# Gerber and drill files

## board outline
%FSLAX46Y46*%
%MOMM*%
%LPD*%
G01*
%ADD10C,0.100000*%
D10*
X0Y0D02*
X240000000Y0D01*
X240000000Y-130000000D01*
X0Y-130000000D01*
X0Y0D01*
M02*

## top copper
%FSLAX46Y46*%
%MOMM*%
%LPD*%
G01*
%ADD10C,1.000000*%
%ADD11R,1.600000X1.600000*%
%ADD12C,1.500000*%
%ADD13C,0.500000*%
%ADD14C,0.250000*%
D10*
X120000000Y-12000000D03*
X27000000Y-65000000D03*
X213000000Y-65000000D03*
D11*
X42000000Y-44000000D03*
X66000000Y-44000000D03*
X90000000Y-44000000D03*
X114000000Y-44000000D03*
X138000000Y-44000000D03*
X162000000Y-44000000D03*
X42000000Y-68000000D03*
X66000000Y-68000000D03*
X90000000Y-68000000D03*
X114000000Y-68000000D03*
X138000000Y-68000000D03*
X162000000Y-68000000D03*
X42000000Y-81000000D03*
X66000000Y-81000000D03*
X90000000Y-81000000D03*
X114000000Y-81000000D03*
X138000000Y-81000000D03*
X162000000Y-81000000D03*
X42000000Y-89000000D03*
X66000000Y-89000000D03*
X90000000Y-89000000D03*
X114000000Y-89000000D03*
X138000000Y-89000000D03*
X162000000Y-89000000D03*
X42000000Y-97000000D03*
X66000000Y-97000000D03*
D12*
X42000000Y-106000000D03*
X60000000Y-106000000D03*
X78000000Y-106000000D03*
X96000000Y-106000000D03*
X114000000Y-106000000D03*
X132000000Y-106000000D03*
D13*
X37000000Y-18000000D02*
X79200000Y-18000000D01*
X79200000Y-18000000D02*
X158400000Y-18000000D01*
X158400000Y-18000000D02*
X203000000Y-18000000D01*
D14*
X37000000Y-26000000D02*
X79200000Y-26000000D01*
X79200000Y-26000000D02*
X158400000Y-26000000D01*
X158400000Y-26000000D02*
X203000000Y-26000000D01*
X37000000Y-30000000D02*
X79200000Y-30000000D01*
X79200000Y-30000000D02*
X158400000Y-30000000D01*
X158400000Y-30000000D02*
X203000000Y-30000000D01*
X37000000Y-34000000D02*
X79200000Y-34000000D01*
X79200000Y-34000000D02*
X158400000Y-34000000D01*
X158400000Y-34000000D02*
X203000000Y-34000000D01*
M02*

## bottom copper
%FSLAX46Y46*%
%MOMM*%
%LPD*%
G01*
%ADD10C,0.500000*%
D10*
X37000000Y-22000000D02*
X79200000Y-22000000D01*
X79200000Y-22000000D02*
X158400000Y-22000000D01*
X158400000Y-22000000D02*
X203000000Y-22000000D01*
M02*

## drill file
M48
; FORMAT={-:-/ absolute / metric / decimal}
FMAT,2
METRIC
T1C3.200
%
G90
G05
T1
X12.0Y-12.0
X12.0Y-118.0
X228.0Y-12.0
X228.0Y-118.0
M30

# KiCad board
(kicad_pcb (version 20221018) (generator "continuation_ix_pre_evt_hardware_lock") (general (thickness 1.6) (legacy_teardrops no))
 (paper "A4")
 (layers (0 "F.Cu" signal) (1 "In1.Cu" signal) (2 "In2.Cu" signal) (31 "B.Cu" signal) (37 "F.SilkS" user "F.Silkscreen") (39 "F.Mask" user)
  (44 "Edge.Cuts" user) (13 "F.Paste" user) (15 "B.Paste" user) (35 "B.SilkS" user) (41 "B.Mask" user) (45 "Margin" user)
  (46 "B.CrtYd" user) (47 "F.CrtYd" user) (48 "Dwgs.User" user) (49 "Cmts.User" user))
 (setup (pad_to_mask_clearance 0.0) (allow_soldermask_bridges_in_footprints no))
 (gr_rect (start 0 0) (end 240.0 130.0) (stroke (width 0.1) (type default)) (fill none) (layer "Edge.Cuts"))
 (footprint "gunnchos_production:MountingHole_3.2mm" (layer "F.Cu") (at 12.0 12.0)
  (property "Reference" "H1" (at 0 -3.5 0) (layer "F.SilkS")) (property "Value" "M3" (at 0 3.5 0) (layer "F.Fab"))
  (pad "" np_thru_hole circle (at 0 0) (size 3.2 3.2) (drill 3.2) (layers "*.Cu" "*.Mask")))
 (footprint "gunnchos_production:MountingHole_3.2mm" (layer "F.Cu") (at 228.0 12.0)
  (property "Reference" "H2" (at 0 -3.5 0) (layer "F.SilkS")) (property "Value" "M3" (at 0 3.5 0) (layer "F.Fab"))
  (pad "" np_thru_hole circle (at 0 0) (size 3.2 3.2) (drill 3.2) (layers "*.Cu" "*.Mask")))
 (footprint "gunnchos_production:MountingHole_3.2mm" (layer "F.Cu") (at 12.0 118.0)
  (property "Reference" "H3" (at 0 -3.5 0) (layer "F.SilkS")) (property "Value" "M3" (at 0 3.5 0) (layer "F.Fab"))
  (pad "" np_thru_hole circle (at 0 0) (size 3.2 3.2) (drill 3.2) (layers "*.Cu" "*.Mask")))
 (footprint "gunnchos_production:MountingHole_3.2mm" (layer "F.Cu") (at 228.0 118.0)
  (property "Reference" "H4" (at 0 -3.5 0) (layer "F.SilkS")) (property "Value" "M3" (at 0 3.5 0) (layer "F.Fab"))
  (pad "" np_thru_hole circle (at 0 0) (size 3.2 3.2) (drill 3.2) (layers "*.Cu" "*.Mask")))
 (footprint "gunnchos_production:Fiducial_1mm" (layer "F.Cu") (at 120.0 12.0)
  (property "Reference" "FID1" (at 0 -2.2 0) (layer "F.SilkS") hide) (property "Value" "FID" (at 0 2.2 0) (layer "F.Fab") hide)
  (pad "1" smd circle (at 0 0) (size 1 1) (layers "F.Cu") (solder_mask_margin 0.5)))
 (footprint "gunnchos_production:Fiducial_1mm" (layer "F.Cu") (at 27.0 65.0)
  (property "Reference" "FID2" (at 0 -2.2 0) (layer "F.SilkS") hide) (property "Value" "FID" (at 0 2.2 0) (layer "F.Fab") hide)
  (pad "1" smd circle (at 0 0) (size 1 1) (layers "F.Cu") (solder_mask_margin 0.5)))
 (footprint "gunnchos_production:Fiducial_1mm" (layer "F.Cu") (at 213.0 65.0)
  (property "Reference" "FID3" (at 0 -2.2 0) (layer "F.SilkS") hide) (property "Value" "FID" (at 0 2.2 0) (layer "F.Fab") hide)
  (pad "1" smd circle (at 0 0) (size 1 1) (layers "F.Cu") (solder_mask_margin 0.5)))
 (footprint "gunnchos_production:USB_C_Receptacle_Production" (layer "F.Cu") (at 42.00 44.00)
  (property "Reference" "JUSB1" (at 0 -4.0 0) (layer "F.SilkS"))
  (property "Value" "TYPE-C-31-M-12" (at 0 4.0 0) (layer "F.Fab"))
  (pad "1" smd rect (at 0 0) (size 1.6 1.6) (layers "F.Cu" "F.Paste" "F.Mask")))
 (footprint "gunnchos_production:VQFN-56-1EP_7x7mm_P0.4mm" (layer "F.Cu") (at 66.00 44.00)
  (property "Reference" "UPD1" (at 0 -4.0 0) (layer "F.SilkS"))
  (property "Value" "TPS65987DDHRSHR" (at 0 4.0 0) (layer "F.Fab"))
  (pad "1" smd rect (at 0 0) (size 1.6 1.6) (layers "F.Cu" "F.Paste" "F.Mask")))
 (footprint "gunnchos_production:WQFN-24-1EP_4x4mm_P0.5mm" (layer "F.Cu") (at 90.00 44.00)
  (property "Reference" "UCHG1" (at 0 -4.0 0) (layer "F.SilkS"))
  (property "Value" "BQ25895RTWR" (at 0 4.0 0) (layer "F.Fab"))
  (pad "1" smd rect (at 0 0) (size 1.6 1.6) (layers "F.Cu" "F.Paste" "F.Mask")))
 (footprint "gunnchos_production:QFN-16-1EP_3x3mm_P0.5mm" (layer "F.Cu") (at 114.00 44.00)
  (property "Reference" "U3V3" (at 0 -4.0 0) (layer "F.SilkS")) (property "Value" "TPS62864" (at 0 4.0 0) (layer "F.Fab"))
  (pad "1" smd rect (at 0 0) (size 1.6 1.6) (layers "F.Cu" "F.Paste" "F.Mask")))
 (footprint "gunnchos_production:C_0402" (layer "F.Cu") (at 138.00 44.00) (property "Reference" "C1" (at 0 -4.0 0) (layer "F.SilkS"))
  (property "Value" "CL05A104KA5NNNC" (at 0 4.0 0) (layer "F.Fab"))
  (pad "1" smd rect (at 0 0) (size 1.6 1.6) (layers "F.Cu" "F.Paste" "F.Mask")))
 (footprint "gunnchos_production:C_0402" (layer "F.Cu") (at 162.00 44.00) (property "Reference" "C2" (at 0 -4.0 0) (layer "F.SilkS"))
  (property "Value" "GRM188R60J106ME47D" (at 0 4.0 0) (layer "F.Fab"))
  (pad "1" smd rect (at 0 0) (size 1.6 1.6) (layers "F.Cu" "F.Paste" "F.Mask")))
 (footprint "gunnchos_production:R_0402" (layer "F.Cu") (at 42.00 68.00) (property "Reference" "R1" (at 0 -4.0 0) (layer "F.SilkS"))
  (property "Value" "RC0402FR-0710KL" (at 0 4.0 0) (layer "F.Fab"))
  (pad "1" smd rect (at 0 0) (size 1.6 1.6) (layers "F.Cu" "F.Paste" "F.Mask")))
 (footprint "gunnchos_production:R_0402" (layer "F.Cu") (at 66.00 68.00) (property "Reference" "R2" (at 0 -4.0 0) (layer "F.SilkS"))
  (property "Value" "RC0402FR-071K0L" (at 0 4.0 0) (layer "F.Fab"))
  (pad "1" smd rect (at 0 0) (size 1.6 1.6) (layers "F.Cu" "F.Paste" "F.Mask")))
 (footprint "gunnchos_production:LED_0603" (layer "F.Cu") (at 90.00 68.00) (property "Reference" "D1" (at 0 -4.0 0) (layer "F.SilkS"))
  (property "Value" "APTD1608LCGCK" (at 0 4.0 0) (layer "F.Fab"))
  (pad "1" smd rect (at 0 0) (size 1.6 1.6) (layers "F.Cu" "F.Paste" "F.Mask")))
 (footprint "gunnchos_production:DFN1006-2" (layer "F.Cu") (at 114.00 68.00)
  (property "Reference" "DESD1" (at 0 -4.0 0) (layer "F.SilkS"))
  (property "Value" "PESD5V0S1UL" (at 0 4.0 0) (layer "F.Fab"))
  (pad "1" smd rect (at 0 0) (size 1.6 1.6) (layers "F.Cu" "F.Paste" "F.Mask")))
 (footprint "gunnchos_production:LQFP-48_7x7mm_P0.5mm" (layer "F.Cu") (at 138.00 68.00)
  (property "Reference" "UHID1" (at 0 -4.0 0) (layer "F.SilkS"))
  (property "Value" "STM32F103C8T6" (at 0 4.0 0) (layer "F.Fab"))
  (pad "1" smd rect (at 0 0) (size 1.6 1.6) (layers "F.Cu" "F.Paste" "F.Mask")))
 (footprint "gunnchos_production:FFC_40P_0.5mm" (layer "F.Cu") (at 162.00 68.00)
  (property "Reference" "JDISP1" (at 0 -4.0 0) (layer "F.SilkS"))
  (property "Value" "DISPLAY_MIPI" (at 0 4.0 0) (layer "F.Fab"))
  (pad "1" smd rect (at 0 0) (size 1.6 1.6) (layers "F.Cu" "F.Paste" "F.Mask")))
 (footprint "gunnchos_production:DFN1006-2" (layer "F.Cu") (at 42.00 81.00)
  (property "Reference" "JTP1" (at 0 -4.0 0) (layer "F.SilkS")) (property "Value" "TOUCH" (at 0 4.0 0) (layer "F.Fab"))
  (pad "1" smd rect (at 0 0) (size 1.6 1.6) (layers "F.Cu" "F.Paste" "F.Mask")))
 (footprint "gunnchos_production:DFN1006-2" (layer "F.Cu") (at 66.00 81.00)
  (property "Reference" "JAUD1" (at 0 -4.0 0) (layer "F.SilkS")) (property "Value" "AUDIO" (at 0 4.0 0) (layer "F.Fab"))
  (pad "1" smd rect (at 0 0) (size 1.6 1.6) (layers "F.Cu" "F.Paste" "F.Mask")))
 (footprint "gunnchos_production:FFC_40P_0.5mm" (layer "F.Cu") (at 90.00 81.00)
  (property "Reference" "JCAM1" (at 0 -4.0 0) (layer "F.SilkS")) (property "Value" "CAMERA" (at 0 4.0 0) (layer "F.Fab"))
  (pad "1" smd rect (at 0 0) (size 1.6 1.6) (layers "F.Cu" "F.Paste" "F.Mask")))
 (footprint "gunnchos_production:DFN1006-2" (layer "F.Cu") (at 114.00 81.00)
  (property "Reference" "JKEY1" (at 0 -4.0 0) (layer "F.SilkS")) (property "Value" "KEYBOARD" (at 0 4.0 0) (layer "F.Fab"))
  (pad "1" smd rect (at 0 0) (size 1.6 1.6) (layers "F.Cu" "F.Paste" "F.Mask")))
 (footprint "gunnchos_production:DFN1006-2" (layer "F.Cu") (at 138.00 81.00)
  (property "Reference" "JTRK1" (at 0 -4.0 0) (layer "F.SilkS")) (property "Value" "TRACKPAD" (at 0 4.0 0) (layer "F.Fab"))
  (pad "1" smd rect (at 0 0) (size 1.6 1.6) (layers "F.Cu" "F.Paste" "F.Mask")))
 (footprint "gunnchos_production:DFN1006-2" (layer "F.Cu") (at 162.00 81.00)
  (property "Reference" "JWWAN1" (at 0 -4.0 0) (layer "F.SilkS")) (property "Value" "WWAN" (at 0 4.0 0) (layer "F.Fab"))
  (pad "1" smd rect (at 0 0) (size 1.6 1.6) (layers "F.Cu" "F.Paste" "F.Mask")))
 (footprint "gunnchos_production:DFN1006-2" (layer "F.Cu") (at 42.00 89.00)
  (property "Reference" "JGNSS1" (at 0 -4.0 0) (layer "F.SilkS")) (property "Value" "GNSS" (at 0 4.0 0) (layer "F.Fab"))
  (pad "1" smd rect (at 0 0) (size 1.6 1.6) (layers "F.Cu" "F.Paste" "F.Mask")))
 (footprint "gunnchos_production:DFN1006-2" (layer "F.Cu") (at 66.00 89.00)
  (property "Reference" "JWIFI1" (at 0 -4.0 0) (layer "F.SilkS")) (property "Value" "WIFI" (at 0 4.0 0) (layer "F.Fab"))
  (pad "1" smd rect (at 0 0) (size 1.6 1.6) (layers "F.Cu" "F.Paste" "F.Mask")))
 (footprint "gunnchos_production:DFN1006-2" (layer "F.Cu") (at 90.00 89.00)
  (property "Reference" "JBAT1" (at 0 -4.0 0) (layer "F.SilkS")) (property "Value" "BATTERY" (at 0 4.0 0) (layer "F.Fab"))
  (pad "1" smd rect (at 0 0) (size 1.6 1.6) (layers "F.Cu" "F.Paste" "F.Mask")))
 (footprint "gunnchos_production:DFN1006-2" (layer "F.Cu") (at 114.00 89.00)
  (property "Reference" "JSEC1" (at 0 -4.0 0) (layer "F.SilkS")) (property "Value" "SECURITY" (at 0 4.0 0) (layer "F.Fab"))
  (pad "1" smd rect (at 0 0) (size 1.6 1.6) (layers "F.Cu" "F.Paste" "F.Mask")))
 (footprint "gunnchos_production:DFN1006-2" (layer "F.Cu") (at 138.00 89.00)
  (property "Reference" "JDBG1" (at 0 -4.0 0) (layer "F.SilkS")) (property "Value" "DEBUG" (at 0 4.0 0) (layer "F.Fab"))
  (pad "1" smd rect (at 0 0) (size 1.6 1.6) (layers "F.Cu" "F.Paste" "F.Mask")))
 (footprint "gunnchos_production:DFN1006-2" (layer "F.Cu") (at 162.00 89.00)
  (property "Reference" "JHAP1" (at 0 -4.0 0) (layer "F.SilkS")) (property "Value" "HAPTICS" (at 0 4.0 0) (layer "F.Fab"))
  (pad "1" smd rect (at 0 0) (size 1.6 1.6) (layers "F.Cu" "F.Paste" "F.Mask")))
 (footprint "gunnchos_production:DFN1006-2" (layer "F.Cu") (at 42.00 97.00)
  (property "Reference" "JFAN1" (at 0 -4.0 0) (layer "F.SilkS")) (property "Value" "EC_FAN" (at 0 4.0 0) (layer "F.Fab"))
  (pad "1" smd rect (at 0 0) (size 1.6 1.6) (layers "F.Cu" "F.Paste" "F.Mask")))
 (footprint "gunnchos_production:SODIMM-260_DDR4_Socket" (layer "F.Cu") (at 66.00 97.00)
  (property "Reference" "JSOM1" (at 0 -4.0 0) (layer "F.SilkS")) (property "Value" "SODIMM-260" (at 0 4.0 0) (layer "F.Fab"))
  (pad "1" smd rect (at 0 0) (size 1.6 1.6) (layers "F.Cu" "F.Paste" "F.Mask")))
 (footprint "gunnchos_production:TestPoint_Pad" (layer "F.Cu") (at 42.0 106.0) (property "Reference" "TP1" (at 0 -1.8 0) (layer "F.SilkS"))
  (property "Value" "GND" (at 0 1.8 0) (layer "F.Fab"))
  (pad "1" smd circle (at 0 0) (size 1.5 1.5) (layers "F.Cu" "F.Mask")))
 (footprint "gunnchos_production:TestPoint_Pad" (layer "F.Cu") (at 60.0 106.0) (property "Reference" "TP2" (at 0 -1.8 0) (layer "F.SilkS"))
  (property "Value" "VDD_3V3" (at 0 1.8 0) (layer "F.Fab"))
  (pad "1" smd circle (at 0 0) (size 1.5 1.5) (layers "F.Cu" "F.Mask")))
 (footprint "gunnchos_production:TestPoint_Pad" (layer "F.Cu") (at 78.0 106.0) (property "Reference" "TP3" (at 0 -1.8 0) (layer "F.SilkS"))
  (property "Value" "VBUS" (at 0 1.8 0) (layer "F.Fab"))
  (pad "1" smd circle (at 0 0) (size 1.5 1.5) (layers "F.Cu" "F.Mask")))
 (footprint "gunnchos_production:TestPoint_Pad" (layer "F.Cu") (at 96.0 106.0) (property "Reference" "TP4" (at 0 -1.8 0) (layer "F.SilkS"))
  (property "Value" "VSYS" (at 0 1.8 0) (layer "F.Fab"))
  (pad "1" smd circle (at 0 0) (size 1.5 1.5) (layers "F.Cu" "F.Mask")))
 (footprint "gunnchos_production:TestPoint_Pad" (layer "F.Cu") (at 114.0 106.0) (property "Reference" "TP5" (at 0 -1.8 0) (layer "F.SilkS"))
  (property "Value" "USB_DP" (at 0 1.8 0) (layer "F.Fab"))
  (pad "1" smd circle (at 0 0) (size 1.5 1.5) (layers "F.Cu" "F.Mask")))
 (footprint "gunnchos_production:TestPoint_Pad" (layer "F.Cu") (at 132.0 106.0) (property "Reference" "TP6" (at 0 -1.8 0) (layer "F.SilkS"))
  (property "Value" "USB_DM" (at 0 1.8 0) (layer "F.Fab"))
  (pad "1" smd circle (at 0 0) (size 1.5 1.5) (layers "F.Cu" "F.Mask")))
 (segment (start 37.00 18.00) (end 79.20 18.00) (width 0.5) (layer "F.Cu") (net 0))
 (segment (start 79.20 18.00) (end 158.40 18.00) (width 0.5) (layer "F.Cu") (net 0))
 (segment (start 158.40 18.00) (end 203.00 18.00) (width 0.5) (layer "F.Cu") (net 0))
 (segment (start 37.00 22.00) (end 79.20 22.00) (width 0.5) (layer "B.Cu") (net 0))
 (segment (start 79.20 22.00) (end 158.40 22.00) (width 0.5) (layer "B.Cu") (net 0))
 (segment (start 158.40 22.00) (end 203.00 22.00) (width 0.5) (layer "B.Cu") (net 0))
 (segment (start 37.00 26.00) (end 79.20 26.00) (width 0.25) (layer "F.Cu") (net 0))
 (segment (start 79.20 26.00) (end 158.40 26.00) (width 0.25) (layer "F.Cu") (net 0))
 (segment (start 158.40 26.00) (end 203.00 26.00) (width 0.25) (layer "F.Cu") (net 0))
 (segment (start 37.00 30.00) (end 79.20 30.00) (width 0.25) (layer "F.Cu") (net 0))
 (segment (start 79.20 30.00) (end 158.40 30.00) (width 0.25) (layer "F.Cu") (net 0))
 (segment (start 158.40 30.00) (end 203.00 30.00) (width 0.25) (layer "F.Cu") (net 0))
 (segment (start 37.00 34.00) (end 79.20 34.00) (width 0.25) (layer "F.Cu") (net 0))
 (segment (start 79.20 34.00) (end 158.40 34.00) (width 0.25) (layer "F.Cu") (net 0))
 (segment (start 158.40 34.00) (end 203.00 34.00) (width 0.25) (layer "F.Cu") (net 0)))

